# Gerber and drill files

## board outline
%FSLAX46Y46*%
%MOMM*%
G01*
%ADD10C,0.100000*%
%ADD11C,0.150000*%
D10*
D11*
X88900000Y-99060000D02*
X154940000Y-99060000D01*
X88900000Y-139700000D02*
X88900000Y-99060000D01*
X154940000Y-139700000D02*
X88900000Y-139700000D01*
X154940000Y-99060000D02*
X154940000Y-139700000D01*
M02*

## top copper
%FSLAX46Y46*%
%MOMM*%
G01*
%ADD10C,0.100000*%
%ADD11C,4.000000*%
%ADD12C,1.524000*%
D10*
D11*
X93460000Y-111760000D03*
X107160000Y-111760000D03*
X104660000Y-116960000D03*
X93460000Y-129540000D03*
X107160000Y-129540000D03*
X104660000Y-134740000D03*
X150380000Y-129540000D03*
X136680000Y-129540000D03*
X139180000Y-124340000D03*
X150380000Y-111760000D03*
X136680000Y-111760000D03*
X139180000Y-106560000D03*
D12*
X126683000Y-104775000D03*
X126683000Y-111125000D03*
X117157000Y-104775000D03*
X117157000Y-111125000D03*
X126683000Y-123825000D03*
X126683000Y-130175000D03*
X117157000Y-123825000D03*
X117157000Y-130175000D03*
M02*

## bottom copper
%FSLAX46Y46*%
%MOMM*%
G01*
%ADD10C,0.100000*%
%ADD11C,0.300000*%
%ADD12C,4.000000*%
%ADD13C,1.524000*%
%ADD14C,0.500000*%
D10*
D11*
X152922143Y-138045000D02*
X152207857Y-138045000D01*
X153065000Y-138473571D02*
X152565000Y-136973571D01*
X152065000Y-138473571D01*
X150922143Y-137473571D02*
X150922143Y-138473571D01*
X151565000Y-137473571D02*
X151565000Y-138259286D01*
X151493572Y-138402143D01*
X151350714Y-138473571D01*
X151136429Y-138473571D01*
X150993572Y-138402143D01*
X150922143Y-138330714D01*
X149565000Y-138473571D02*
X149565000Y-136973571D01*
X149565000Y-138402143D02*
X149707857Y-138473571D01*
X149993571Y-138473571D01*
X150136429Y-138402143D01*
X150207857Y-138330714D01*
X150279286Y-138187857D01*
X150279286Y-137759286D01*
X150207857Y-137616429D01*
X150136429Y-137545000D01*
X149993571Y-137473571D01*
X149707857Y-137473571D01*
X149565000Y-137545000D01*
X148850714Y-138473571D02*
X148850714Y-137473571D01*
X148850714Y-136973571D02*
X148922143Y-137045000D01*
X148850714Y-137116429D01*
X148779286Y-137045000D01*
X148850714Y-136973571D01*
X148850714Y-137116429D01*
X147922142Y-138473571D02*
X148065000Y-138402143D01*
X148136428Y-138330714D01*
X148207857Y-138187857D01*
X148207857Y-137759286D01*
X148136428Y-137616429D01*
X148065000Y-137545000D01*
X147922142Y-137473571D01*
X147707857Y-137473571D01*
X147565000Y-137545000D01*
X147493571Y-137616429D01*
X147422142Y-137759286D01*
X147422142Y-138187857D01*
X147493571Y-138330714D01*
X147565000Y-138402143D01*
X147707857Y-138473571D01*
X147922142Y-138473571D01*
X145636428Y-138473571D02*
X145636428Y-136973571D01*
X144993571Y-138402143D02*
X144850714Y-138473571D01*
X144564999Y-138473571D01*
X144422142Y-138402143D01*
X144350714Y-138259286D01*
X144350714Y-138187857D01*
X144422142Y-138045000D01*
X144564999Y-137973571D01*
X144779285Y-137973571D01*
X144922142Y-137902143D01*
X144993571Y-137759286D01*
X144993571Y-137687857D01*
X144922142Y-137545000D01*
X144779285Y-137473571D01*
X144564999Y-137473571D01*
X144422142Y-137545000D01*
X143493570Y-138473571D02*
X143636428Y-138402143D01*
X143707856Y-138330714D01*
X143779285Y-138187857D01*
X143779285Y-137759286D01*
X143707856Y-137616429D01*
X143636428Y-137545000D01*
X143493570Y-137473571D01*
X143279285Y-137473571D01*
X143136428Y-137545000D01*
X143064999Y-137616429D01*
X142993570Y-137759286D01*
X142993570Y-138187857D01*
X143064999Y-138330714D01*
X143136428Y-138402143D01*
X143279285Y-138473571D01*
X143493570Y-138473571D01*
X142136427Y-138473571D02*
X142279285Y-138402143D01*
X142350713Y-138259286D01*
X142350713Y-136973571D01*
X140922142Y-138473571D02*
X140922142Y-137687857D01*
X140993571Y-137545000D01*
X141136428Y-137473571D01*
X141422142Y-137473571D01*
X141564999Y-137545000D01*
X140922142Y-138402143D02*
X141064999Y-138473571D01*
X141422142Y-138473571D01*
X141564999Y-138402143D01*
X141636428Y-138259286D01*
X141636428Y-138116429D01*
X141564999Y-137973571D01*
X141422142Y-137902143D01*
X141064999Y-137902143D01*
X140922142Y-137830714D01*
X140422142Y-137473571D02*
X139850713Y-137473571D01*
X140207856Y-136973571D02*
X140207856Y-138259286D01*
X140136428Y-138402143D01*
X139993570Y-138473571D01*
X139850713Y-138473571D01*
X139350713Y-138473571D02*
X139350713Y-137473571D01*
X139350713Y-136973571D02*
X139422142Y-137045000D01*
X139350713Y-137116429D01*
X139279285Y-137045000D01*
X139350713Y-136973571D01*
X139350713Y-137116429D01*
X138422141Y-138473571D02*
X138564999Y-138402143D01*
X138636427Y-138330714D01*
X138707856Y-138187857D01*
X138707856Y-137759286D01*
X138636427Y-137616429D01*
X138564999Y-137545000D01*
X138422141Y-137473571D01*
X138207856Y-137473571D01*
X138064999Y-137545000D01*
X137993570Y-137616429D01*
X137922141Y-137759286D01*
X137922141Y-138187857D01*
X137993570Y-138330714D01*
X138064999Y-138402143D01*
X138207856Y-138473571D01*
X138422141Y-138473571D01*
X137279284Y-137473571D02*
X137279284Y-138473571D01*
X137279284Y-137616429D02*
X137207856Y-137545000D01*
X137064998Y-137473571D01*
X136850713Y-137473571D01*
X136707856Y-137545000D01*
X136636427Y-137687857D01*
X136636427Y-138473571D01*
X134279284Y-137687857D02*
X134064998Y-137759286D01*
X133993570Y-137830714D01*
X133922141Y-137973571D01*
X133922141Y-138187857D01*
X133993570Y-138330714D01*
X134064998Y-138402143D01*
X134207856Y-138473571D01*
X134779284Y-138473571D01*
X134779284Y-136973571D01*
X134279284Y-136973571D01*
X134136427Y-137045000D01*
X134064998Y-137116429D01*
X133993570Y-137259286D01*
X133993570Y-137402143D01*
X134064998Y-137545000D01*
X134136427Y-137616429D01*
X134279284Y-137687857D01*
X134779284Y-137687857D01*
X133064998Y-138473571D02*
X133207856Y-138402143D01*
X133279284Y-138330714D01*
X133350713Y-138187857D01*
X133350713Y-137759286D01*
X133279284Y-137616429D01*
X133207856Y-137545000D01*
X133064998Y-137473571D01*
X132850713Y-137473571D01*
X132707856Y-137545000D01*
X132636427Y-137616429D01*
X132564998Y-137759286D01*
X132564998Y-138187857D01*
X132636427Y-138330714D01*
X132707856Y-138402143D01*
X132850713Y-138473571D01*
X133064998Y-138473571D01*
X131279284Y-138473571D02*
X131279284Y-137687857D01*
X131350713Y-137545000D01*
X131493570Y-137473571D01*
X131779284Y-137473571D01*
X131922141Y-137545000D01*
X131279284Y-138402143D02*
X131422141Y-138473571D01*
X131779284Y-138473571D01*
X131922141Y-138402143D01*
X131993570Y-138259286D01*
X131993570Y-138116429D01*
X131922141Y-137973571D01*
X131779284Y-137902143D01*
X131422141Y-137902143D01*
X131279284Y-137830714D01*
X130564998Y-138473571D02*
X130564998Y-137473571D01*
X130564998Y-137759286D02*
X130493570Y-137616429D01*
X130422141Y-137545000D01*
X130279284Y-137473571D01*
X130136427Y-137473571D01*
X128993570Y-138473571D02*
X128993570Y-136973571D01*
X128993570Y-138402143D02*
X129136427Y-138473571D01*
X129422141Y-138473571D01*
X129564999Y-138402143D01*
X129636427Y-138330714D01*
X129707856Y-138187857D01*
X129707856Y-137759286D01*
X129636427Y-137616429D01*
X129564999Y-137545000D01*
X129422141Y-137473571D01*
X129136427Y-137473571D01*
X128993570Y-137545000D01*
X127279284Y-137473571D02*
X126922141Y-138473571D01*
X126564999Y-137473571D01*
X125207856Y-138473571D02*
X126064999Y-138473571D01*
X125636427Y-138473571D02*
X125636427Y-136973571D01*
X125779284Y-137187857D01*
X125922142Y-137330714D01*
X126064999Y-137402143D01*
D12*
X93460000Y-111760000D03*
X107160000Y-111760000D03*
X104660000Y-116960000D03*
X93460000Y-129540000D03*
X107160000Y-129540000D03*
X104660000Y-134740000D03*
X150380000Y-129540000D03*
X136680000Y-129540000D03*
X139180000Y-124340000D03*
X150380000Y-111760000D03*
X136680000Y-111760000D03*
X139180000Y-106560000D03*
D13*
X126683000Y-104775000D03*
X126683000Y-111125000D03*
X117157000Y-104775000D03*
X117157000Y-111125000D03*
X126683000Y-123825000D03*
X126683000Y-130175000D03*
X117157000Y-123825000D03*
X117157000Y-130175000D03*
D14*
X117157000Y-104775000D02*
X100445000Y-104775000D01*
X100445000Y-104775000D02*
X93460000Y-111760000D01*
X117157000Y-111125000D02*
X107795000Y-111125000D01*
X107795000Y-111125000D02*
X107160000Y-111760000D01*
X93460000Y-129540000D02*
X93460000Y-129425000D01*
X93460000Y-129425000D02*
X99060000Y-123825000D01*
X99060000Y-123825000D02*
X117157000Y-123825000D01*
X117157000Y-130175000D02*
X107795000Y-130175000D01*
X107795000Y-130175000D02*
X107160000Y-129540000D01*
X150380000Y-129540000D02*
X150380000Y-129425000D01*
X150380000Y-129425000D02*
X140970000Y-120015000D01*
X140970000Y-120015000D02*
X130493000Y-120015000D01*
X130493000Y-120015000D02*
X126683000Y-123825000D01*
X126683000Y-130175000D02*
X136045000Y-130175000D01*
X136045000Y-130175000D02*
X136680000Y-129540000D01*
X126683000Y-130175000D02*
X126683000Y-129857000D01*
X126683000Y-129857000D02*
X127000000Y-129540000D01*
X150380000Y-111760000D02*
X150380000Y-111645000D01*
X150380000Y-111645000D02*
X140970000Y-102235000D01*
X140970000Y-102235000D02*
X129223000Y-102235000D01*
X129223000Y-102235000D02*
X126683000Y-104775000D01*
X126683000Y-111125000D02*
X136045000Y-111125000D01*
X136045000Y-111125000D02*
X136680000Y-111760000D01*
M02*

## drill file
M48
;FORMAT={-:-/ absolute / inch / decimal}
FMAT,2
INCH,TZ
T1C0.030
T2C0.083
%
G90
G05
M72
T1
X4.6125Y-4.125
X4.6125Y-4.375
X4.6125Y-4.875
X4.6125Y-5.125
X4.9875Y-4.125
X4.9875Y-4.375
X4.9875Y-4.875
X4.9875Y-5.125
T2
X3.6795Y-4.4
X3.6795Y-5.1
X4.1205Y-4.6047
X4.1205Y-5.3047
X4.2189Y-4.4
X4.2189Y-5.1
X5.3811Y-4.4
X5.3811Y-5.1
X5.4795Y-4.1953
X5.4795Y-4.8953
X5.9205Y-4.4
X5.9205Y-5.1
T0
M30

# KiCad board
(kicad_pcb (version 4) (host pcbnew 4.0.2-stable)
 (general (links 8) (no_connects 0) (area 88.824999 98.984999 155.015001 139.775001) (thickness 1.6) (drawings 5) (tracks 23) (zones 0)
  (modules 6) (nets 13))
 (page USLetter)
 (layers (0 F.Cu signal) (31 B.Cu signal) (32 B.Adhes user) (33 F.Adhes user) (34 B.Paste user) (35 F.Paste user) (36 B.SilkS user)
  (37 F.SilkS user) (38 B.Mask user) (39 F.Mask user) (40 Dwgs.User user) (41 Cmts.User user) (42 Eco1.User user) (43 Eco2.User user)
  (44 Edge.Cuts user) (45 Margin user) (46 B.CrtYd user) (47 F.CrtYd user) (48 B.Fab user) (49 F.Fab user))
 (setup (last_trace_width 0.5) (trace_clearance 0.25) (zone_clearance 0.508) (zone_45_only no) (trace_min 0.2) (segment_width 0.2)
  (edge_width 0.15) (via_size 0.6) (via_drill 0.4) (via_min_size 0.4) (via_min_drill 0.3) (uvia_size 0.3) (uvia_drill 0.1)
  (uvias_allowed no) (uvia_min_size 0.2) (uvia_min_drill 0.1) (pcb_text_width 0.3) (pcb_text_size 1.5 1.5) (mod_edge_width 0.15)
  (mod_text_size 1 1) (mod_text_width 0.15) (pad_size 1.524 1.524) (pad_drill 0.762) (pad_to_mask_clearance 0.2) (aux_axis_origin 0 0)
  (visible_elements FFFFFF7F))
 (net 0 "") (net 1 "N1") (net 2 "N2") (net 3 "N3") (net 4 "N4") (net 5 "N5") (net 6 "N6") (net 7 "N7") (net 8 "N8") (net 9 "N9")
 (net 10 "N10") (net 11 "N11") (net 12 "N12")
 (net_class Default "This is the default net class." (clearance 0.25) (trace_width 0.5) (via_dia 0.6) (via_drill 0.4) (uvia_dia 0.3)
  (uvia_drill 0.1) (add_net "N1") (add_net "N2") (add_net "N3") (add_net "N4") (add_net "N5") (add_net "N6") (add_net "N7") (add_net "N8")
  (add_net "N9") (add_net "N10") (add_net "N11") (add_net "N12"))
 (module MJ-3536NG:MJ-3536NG (layer F.Cu) (at 99.06 111.76)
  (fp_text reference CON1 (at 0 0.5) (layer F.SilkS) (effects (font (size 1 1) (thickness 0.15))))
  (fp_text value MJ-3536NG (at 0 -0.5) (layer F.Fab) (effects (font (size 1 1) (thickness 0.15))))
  (pad 1 thru_hole circle (at -5.6 0) (size 4 4) (drill 2.1) (layers *.Cu *.Mask F.SilkS) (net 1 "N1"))
  (pad 2 thru_hole circle (at 8.1 0) (size 4 4) (drill 2.1) (layers *.Cu *.Mask F.SilkS) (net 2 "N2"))
  (pad 3 thru_hole circle (at 5.6 5.2) (size 4 4) (drill 2.1) (layers *.Cu *.Mask F.SilkS) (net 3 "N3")))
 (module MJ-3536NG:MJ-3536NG (layer F.Cu) (at 99.06 129.54)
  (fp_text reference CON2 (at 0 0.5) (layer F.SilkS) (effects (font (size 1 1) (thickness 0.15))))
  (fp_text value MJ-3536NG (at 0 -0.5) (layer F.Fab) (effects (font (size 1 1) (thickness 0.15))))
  (pad 1 thru_hole circle (at -5.6 0) (size 4 4) (drill 2.1) (layers *.Cu *.Mask F.SilkS) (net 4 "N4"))
  (pad 2 thru_hole circle (at 8.1 0) (size 4 4) (drill 2.1) (layers *.Cu *.Mask F.SilkS) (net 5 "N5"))
  (pad 3 thru_hole circle (at 5.6 5.2) (size 4 4) (drill 2.1) (layers *.Cu *.Mask F.SilkS) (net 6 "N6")))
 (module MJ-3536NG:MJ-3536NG (layer F.Cu) (at 144.78 129.54 180)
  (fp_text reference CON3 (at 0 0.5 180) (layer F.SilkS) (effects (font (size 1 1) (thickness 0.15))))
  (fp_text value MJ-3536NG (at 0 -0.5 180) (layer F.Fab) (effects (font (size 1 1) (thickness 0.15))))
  (pad 1 thru_hole circle (at -5.6 0 180) (size 4 4) (drill 2.1) (layers *.Cu *.Mask F.SilkS) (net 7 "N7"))
  (pad 2 thru_hole circle (at 8.1 0 180) (size 4 4) (drill 2.1) (layers *.Cu *.Mask F.SilkS) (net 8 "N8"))
  (pad 3 thru_hole circle (at 5.6 5.2 180) (size 4 4) (drill 2.1) (layers *.Cu *.Mask F.SilkS) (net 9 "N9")))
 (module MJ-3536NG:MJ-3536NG (layer F.Cu) (at 144.78 111.76 180)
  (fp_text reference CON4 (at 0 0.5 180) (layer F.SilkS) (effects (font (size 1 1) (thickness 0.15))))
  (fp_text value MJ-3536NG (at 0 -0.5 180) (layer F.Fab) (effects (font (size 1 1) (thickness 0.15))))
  (pad 1 thru_hole circle (at -5.6 0 180) (size 4 4) (drill 2.1) (layers *.Cu *.Mask F.SilkS) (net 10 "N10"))
  (pad 2 thru_hole circle (at 8.1 0 180) (size 4 4) (drill 2.1) (layers *.Cu *.Mask F.SilkS) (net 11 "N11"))
  (pad 3 thru_hole circle (at 5.6 5.2 180) (size 4 4) (drill 2.1) (layers *.Cu *.Mask F.SilkS) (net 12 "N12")))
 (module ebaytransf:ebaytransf (layer F.Cu) (at 121.92 107.95)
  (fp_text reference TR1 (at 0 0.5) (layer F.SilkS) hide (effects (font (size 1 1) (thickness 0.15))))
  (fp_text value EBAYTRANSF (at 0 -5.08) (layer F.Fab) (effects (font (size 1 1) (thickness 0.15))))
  (pad 4 thru_hole circle (at 4.763 -3.175) (size 1.524 1.524) (drill 0.762) (layers *.Cu *.Mask F.SilkS) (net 10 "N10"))
  (pad 3 thru_hole circle (at 4.763 3.175) (size 1.524 1.524) (drill 0.762) (layers *.Cu *.Mask F.SilkS) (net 11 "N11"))
  (pad 1 thru_hole circle (at -4.763 -3.175) (size 1.524 1.524) (drill 0.762) (layers *.Cu *.Mask F.SilkS) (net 1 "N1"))
  (pad 2 thru_hole circle (at -4.763 3.175) (size 1.524 1.524) (drill 0.762) (layers *.Cu *.Mask F.SilkS) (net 2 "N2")))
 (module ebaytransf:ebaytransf (layer F.Cu) (at 121.92 127)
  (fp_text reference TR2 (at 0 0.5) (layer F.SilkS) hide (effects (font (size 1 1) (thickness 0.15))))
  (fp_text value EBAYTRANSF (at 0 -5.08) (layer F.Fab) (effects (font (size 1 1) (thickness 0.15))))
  (pad 4 thru_hole circle (at 4.763 -3.175) (size 1.524 1.524) (drill 0.762) (layers *.Cu *.Mask F.SilkS) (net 7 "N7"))
  (pad 3 thru_hole circle (at 4.763 3.175) (size 1.524 1.524) (drill 0.762) (layers *.Cu *.Mask F.SilkS) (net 8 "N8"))
  (pad 1 thru_hole circle (at -4.763 -3.175) (size 1.524 1.524) (drill 0.762) (layers *.Cu *.Mask F.SilkS) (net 4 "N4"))
  (pad 2 thru_hole circle (at -4.763 3.175) (size 1.524 1.524) (drill 0.762) (layers *.Cu *.Mask F.SilkS) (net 5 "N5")))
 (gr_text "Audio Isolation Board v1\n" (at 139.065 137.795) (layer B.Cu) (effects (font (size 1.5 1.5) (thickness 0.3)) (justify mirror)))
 (gr_line (start 88.9 99.06) (end 154.94 99.06) (angle 90) (layer Edge.Cuts) (width 0.15))
 (gr_line (start 88.9 139.7) (end 88.9 99.06) (angle 90) (layer Edge.Cuts) (width 0.15))
 (gr_line (start 154.94 139.7) (end 88.9 139.7) (angle 90) (layer Edge.Cuts) (width 0.15))
 (gr_line (start 154.94 99.06) (end 154.94 139.7) (angle 90) (layer Edge.Cuts) (width 0.15))
 (segment (start 117.157 104.775) (end 100.445 104.775) (width 0.5) (layer B.Cu) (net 1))
 (segment (start 100.445 104.775) (end 93.46 111.76) (width 0.5) (layer B.Cu) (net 1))
 (segment (start 117.157 111.125) (end 107.795 111.125) (width 0.5) (layer B.Cu) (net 2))
 (segment (start 107.795 111.125) (end 107.16 111.76) (width 0.5) (layer B.Cu) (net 2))
 (segment (start 93.46 129.54) (end 93.46 129.425) (width 0.5) (layer B.Cu) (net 4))
 (segment (start 93.46 129.425) (end 99.06 123.825) (width 0.5) (layer B.Cu) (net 4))
 (segment (start 99.06 123.825) (end 117.157 123.825) (width 0.5) (layer B.Cu) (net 4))
 (segment (start 117.157 130.175) (end 107.795 130.175) (width 0.5) (layer B.Cu) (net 5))
 (segment (start 107.795 130.175) (end 107.16 129.54) (width 0.5) (layer B.Cu) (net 5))
 (segment (start 150.38 129.54) (end 150.38 129.425) (width 0.5) (layer B.Cu) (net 7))
 (segment (start 150.38 129.425) (end 140.97 120.015) (width 0.5) (layer B.Cu) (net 7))
 (segment (start 140.97 120.015) (end 130.493 120.015) (width 0.5) (layer B.Cu) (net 7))
 (segment (start 130.493 120.015) (end 126.683 123.825) (width 0.5) (layer B.Cu) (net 7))
 (segment (start 126.683 130.175) (end 136.045 130.175) (width 0.5) (layer B.Cu) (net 8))
 (segment (start 136.045 130.175) (end 136.68 129.54) (width 0.5) (layer B.Cu) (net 8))
 (segment (start 126.683 130.175) (end 126.683 129.857) (width 0.5) (layer B.Cu) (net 8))
 (segment (start 126.683 129.857) (end 127 129.54) (width 0.5) (layer B.Cu) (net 8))
 (segment (start 150.38 111.76) (end 150.38 111.645) (width 0.5) (layer B.Cu) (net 10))
 (segment (start 150.38 111.645) (end 140.97 102.235) (width 0.5) (layer B.Cu) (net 10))
 (segment (start 140.97 102.235) (end 129.223 102.235) (width 0.5) (layer B.Cu) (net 10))
 (segment (start 129.223 102.235) (end 126.683 104.775) (width 0.5) (layer B.Cu) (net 10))
 (segment (start 126.683 111.125) (end 136.045 111.125) (width 0.5) (layer B.Cu) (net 11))
 (segment (start 136.045 111.125) (end 136.68 111.76) (width 0.5) (layer B.Cu) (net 11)))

